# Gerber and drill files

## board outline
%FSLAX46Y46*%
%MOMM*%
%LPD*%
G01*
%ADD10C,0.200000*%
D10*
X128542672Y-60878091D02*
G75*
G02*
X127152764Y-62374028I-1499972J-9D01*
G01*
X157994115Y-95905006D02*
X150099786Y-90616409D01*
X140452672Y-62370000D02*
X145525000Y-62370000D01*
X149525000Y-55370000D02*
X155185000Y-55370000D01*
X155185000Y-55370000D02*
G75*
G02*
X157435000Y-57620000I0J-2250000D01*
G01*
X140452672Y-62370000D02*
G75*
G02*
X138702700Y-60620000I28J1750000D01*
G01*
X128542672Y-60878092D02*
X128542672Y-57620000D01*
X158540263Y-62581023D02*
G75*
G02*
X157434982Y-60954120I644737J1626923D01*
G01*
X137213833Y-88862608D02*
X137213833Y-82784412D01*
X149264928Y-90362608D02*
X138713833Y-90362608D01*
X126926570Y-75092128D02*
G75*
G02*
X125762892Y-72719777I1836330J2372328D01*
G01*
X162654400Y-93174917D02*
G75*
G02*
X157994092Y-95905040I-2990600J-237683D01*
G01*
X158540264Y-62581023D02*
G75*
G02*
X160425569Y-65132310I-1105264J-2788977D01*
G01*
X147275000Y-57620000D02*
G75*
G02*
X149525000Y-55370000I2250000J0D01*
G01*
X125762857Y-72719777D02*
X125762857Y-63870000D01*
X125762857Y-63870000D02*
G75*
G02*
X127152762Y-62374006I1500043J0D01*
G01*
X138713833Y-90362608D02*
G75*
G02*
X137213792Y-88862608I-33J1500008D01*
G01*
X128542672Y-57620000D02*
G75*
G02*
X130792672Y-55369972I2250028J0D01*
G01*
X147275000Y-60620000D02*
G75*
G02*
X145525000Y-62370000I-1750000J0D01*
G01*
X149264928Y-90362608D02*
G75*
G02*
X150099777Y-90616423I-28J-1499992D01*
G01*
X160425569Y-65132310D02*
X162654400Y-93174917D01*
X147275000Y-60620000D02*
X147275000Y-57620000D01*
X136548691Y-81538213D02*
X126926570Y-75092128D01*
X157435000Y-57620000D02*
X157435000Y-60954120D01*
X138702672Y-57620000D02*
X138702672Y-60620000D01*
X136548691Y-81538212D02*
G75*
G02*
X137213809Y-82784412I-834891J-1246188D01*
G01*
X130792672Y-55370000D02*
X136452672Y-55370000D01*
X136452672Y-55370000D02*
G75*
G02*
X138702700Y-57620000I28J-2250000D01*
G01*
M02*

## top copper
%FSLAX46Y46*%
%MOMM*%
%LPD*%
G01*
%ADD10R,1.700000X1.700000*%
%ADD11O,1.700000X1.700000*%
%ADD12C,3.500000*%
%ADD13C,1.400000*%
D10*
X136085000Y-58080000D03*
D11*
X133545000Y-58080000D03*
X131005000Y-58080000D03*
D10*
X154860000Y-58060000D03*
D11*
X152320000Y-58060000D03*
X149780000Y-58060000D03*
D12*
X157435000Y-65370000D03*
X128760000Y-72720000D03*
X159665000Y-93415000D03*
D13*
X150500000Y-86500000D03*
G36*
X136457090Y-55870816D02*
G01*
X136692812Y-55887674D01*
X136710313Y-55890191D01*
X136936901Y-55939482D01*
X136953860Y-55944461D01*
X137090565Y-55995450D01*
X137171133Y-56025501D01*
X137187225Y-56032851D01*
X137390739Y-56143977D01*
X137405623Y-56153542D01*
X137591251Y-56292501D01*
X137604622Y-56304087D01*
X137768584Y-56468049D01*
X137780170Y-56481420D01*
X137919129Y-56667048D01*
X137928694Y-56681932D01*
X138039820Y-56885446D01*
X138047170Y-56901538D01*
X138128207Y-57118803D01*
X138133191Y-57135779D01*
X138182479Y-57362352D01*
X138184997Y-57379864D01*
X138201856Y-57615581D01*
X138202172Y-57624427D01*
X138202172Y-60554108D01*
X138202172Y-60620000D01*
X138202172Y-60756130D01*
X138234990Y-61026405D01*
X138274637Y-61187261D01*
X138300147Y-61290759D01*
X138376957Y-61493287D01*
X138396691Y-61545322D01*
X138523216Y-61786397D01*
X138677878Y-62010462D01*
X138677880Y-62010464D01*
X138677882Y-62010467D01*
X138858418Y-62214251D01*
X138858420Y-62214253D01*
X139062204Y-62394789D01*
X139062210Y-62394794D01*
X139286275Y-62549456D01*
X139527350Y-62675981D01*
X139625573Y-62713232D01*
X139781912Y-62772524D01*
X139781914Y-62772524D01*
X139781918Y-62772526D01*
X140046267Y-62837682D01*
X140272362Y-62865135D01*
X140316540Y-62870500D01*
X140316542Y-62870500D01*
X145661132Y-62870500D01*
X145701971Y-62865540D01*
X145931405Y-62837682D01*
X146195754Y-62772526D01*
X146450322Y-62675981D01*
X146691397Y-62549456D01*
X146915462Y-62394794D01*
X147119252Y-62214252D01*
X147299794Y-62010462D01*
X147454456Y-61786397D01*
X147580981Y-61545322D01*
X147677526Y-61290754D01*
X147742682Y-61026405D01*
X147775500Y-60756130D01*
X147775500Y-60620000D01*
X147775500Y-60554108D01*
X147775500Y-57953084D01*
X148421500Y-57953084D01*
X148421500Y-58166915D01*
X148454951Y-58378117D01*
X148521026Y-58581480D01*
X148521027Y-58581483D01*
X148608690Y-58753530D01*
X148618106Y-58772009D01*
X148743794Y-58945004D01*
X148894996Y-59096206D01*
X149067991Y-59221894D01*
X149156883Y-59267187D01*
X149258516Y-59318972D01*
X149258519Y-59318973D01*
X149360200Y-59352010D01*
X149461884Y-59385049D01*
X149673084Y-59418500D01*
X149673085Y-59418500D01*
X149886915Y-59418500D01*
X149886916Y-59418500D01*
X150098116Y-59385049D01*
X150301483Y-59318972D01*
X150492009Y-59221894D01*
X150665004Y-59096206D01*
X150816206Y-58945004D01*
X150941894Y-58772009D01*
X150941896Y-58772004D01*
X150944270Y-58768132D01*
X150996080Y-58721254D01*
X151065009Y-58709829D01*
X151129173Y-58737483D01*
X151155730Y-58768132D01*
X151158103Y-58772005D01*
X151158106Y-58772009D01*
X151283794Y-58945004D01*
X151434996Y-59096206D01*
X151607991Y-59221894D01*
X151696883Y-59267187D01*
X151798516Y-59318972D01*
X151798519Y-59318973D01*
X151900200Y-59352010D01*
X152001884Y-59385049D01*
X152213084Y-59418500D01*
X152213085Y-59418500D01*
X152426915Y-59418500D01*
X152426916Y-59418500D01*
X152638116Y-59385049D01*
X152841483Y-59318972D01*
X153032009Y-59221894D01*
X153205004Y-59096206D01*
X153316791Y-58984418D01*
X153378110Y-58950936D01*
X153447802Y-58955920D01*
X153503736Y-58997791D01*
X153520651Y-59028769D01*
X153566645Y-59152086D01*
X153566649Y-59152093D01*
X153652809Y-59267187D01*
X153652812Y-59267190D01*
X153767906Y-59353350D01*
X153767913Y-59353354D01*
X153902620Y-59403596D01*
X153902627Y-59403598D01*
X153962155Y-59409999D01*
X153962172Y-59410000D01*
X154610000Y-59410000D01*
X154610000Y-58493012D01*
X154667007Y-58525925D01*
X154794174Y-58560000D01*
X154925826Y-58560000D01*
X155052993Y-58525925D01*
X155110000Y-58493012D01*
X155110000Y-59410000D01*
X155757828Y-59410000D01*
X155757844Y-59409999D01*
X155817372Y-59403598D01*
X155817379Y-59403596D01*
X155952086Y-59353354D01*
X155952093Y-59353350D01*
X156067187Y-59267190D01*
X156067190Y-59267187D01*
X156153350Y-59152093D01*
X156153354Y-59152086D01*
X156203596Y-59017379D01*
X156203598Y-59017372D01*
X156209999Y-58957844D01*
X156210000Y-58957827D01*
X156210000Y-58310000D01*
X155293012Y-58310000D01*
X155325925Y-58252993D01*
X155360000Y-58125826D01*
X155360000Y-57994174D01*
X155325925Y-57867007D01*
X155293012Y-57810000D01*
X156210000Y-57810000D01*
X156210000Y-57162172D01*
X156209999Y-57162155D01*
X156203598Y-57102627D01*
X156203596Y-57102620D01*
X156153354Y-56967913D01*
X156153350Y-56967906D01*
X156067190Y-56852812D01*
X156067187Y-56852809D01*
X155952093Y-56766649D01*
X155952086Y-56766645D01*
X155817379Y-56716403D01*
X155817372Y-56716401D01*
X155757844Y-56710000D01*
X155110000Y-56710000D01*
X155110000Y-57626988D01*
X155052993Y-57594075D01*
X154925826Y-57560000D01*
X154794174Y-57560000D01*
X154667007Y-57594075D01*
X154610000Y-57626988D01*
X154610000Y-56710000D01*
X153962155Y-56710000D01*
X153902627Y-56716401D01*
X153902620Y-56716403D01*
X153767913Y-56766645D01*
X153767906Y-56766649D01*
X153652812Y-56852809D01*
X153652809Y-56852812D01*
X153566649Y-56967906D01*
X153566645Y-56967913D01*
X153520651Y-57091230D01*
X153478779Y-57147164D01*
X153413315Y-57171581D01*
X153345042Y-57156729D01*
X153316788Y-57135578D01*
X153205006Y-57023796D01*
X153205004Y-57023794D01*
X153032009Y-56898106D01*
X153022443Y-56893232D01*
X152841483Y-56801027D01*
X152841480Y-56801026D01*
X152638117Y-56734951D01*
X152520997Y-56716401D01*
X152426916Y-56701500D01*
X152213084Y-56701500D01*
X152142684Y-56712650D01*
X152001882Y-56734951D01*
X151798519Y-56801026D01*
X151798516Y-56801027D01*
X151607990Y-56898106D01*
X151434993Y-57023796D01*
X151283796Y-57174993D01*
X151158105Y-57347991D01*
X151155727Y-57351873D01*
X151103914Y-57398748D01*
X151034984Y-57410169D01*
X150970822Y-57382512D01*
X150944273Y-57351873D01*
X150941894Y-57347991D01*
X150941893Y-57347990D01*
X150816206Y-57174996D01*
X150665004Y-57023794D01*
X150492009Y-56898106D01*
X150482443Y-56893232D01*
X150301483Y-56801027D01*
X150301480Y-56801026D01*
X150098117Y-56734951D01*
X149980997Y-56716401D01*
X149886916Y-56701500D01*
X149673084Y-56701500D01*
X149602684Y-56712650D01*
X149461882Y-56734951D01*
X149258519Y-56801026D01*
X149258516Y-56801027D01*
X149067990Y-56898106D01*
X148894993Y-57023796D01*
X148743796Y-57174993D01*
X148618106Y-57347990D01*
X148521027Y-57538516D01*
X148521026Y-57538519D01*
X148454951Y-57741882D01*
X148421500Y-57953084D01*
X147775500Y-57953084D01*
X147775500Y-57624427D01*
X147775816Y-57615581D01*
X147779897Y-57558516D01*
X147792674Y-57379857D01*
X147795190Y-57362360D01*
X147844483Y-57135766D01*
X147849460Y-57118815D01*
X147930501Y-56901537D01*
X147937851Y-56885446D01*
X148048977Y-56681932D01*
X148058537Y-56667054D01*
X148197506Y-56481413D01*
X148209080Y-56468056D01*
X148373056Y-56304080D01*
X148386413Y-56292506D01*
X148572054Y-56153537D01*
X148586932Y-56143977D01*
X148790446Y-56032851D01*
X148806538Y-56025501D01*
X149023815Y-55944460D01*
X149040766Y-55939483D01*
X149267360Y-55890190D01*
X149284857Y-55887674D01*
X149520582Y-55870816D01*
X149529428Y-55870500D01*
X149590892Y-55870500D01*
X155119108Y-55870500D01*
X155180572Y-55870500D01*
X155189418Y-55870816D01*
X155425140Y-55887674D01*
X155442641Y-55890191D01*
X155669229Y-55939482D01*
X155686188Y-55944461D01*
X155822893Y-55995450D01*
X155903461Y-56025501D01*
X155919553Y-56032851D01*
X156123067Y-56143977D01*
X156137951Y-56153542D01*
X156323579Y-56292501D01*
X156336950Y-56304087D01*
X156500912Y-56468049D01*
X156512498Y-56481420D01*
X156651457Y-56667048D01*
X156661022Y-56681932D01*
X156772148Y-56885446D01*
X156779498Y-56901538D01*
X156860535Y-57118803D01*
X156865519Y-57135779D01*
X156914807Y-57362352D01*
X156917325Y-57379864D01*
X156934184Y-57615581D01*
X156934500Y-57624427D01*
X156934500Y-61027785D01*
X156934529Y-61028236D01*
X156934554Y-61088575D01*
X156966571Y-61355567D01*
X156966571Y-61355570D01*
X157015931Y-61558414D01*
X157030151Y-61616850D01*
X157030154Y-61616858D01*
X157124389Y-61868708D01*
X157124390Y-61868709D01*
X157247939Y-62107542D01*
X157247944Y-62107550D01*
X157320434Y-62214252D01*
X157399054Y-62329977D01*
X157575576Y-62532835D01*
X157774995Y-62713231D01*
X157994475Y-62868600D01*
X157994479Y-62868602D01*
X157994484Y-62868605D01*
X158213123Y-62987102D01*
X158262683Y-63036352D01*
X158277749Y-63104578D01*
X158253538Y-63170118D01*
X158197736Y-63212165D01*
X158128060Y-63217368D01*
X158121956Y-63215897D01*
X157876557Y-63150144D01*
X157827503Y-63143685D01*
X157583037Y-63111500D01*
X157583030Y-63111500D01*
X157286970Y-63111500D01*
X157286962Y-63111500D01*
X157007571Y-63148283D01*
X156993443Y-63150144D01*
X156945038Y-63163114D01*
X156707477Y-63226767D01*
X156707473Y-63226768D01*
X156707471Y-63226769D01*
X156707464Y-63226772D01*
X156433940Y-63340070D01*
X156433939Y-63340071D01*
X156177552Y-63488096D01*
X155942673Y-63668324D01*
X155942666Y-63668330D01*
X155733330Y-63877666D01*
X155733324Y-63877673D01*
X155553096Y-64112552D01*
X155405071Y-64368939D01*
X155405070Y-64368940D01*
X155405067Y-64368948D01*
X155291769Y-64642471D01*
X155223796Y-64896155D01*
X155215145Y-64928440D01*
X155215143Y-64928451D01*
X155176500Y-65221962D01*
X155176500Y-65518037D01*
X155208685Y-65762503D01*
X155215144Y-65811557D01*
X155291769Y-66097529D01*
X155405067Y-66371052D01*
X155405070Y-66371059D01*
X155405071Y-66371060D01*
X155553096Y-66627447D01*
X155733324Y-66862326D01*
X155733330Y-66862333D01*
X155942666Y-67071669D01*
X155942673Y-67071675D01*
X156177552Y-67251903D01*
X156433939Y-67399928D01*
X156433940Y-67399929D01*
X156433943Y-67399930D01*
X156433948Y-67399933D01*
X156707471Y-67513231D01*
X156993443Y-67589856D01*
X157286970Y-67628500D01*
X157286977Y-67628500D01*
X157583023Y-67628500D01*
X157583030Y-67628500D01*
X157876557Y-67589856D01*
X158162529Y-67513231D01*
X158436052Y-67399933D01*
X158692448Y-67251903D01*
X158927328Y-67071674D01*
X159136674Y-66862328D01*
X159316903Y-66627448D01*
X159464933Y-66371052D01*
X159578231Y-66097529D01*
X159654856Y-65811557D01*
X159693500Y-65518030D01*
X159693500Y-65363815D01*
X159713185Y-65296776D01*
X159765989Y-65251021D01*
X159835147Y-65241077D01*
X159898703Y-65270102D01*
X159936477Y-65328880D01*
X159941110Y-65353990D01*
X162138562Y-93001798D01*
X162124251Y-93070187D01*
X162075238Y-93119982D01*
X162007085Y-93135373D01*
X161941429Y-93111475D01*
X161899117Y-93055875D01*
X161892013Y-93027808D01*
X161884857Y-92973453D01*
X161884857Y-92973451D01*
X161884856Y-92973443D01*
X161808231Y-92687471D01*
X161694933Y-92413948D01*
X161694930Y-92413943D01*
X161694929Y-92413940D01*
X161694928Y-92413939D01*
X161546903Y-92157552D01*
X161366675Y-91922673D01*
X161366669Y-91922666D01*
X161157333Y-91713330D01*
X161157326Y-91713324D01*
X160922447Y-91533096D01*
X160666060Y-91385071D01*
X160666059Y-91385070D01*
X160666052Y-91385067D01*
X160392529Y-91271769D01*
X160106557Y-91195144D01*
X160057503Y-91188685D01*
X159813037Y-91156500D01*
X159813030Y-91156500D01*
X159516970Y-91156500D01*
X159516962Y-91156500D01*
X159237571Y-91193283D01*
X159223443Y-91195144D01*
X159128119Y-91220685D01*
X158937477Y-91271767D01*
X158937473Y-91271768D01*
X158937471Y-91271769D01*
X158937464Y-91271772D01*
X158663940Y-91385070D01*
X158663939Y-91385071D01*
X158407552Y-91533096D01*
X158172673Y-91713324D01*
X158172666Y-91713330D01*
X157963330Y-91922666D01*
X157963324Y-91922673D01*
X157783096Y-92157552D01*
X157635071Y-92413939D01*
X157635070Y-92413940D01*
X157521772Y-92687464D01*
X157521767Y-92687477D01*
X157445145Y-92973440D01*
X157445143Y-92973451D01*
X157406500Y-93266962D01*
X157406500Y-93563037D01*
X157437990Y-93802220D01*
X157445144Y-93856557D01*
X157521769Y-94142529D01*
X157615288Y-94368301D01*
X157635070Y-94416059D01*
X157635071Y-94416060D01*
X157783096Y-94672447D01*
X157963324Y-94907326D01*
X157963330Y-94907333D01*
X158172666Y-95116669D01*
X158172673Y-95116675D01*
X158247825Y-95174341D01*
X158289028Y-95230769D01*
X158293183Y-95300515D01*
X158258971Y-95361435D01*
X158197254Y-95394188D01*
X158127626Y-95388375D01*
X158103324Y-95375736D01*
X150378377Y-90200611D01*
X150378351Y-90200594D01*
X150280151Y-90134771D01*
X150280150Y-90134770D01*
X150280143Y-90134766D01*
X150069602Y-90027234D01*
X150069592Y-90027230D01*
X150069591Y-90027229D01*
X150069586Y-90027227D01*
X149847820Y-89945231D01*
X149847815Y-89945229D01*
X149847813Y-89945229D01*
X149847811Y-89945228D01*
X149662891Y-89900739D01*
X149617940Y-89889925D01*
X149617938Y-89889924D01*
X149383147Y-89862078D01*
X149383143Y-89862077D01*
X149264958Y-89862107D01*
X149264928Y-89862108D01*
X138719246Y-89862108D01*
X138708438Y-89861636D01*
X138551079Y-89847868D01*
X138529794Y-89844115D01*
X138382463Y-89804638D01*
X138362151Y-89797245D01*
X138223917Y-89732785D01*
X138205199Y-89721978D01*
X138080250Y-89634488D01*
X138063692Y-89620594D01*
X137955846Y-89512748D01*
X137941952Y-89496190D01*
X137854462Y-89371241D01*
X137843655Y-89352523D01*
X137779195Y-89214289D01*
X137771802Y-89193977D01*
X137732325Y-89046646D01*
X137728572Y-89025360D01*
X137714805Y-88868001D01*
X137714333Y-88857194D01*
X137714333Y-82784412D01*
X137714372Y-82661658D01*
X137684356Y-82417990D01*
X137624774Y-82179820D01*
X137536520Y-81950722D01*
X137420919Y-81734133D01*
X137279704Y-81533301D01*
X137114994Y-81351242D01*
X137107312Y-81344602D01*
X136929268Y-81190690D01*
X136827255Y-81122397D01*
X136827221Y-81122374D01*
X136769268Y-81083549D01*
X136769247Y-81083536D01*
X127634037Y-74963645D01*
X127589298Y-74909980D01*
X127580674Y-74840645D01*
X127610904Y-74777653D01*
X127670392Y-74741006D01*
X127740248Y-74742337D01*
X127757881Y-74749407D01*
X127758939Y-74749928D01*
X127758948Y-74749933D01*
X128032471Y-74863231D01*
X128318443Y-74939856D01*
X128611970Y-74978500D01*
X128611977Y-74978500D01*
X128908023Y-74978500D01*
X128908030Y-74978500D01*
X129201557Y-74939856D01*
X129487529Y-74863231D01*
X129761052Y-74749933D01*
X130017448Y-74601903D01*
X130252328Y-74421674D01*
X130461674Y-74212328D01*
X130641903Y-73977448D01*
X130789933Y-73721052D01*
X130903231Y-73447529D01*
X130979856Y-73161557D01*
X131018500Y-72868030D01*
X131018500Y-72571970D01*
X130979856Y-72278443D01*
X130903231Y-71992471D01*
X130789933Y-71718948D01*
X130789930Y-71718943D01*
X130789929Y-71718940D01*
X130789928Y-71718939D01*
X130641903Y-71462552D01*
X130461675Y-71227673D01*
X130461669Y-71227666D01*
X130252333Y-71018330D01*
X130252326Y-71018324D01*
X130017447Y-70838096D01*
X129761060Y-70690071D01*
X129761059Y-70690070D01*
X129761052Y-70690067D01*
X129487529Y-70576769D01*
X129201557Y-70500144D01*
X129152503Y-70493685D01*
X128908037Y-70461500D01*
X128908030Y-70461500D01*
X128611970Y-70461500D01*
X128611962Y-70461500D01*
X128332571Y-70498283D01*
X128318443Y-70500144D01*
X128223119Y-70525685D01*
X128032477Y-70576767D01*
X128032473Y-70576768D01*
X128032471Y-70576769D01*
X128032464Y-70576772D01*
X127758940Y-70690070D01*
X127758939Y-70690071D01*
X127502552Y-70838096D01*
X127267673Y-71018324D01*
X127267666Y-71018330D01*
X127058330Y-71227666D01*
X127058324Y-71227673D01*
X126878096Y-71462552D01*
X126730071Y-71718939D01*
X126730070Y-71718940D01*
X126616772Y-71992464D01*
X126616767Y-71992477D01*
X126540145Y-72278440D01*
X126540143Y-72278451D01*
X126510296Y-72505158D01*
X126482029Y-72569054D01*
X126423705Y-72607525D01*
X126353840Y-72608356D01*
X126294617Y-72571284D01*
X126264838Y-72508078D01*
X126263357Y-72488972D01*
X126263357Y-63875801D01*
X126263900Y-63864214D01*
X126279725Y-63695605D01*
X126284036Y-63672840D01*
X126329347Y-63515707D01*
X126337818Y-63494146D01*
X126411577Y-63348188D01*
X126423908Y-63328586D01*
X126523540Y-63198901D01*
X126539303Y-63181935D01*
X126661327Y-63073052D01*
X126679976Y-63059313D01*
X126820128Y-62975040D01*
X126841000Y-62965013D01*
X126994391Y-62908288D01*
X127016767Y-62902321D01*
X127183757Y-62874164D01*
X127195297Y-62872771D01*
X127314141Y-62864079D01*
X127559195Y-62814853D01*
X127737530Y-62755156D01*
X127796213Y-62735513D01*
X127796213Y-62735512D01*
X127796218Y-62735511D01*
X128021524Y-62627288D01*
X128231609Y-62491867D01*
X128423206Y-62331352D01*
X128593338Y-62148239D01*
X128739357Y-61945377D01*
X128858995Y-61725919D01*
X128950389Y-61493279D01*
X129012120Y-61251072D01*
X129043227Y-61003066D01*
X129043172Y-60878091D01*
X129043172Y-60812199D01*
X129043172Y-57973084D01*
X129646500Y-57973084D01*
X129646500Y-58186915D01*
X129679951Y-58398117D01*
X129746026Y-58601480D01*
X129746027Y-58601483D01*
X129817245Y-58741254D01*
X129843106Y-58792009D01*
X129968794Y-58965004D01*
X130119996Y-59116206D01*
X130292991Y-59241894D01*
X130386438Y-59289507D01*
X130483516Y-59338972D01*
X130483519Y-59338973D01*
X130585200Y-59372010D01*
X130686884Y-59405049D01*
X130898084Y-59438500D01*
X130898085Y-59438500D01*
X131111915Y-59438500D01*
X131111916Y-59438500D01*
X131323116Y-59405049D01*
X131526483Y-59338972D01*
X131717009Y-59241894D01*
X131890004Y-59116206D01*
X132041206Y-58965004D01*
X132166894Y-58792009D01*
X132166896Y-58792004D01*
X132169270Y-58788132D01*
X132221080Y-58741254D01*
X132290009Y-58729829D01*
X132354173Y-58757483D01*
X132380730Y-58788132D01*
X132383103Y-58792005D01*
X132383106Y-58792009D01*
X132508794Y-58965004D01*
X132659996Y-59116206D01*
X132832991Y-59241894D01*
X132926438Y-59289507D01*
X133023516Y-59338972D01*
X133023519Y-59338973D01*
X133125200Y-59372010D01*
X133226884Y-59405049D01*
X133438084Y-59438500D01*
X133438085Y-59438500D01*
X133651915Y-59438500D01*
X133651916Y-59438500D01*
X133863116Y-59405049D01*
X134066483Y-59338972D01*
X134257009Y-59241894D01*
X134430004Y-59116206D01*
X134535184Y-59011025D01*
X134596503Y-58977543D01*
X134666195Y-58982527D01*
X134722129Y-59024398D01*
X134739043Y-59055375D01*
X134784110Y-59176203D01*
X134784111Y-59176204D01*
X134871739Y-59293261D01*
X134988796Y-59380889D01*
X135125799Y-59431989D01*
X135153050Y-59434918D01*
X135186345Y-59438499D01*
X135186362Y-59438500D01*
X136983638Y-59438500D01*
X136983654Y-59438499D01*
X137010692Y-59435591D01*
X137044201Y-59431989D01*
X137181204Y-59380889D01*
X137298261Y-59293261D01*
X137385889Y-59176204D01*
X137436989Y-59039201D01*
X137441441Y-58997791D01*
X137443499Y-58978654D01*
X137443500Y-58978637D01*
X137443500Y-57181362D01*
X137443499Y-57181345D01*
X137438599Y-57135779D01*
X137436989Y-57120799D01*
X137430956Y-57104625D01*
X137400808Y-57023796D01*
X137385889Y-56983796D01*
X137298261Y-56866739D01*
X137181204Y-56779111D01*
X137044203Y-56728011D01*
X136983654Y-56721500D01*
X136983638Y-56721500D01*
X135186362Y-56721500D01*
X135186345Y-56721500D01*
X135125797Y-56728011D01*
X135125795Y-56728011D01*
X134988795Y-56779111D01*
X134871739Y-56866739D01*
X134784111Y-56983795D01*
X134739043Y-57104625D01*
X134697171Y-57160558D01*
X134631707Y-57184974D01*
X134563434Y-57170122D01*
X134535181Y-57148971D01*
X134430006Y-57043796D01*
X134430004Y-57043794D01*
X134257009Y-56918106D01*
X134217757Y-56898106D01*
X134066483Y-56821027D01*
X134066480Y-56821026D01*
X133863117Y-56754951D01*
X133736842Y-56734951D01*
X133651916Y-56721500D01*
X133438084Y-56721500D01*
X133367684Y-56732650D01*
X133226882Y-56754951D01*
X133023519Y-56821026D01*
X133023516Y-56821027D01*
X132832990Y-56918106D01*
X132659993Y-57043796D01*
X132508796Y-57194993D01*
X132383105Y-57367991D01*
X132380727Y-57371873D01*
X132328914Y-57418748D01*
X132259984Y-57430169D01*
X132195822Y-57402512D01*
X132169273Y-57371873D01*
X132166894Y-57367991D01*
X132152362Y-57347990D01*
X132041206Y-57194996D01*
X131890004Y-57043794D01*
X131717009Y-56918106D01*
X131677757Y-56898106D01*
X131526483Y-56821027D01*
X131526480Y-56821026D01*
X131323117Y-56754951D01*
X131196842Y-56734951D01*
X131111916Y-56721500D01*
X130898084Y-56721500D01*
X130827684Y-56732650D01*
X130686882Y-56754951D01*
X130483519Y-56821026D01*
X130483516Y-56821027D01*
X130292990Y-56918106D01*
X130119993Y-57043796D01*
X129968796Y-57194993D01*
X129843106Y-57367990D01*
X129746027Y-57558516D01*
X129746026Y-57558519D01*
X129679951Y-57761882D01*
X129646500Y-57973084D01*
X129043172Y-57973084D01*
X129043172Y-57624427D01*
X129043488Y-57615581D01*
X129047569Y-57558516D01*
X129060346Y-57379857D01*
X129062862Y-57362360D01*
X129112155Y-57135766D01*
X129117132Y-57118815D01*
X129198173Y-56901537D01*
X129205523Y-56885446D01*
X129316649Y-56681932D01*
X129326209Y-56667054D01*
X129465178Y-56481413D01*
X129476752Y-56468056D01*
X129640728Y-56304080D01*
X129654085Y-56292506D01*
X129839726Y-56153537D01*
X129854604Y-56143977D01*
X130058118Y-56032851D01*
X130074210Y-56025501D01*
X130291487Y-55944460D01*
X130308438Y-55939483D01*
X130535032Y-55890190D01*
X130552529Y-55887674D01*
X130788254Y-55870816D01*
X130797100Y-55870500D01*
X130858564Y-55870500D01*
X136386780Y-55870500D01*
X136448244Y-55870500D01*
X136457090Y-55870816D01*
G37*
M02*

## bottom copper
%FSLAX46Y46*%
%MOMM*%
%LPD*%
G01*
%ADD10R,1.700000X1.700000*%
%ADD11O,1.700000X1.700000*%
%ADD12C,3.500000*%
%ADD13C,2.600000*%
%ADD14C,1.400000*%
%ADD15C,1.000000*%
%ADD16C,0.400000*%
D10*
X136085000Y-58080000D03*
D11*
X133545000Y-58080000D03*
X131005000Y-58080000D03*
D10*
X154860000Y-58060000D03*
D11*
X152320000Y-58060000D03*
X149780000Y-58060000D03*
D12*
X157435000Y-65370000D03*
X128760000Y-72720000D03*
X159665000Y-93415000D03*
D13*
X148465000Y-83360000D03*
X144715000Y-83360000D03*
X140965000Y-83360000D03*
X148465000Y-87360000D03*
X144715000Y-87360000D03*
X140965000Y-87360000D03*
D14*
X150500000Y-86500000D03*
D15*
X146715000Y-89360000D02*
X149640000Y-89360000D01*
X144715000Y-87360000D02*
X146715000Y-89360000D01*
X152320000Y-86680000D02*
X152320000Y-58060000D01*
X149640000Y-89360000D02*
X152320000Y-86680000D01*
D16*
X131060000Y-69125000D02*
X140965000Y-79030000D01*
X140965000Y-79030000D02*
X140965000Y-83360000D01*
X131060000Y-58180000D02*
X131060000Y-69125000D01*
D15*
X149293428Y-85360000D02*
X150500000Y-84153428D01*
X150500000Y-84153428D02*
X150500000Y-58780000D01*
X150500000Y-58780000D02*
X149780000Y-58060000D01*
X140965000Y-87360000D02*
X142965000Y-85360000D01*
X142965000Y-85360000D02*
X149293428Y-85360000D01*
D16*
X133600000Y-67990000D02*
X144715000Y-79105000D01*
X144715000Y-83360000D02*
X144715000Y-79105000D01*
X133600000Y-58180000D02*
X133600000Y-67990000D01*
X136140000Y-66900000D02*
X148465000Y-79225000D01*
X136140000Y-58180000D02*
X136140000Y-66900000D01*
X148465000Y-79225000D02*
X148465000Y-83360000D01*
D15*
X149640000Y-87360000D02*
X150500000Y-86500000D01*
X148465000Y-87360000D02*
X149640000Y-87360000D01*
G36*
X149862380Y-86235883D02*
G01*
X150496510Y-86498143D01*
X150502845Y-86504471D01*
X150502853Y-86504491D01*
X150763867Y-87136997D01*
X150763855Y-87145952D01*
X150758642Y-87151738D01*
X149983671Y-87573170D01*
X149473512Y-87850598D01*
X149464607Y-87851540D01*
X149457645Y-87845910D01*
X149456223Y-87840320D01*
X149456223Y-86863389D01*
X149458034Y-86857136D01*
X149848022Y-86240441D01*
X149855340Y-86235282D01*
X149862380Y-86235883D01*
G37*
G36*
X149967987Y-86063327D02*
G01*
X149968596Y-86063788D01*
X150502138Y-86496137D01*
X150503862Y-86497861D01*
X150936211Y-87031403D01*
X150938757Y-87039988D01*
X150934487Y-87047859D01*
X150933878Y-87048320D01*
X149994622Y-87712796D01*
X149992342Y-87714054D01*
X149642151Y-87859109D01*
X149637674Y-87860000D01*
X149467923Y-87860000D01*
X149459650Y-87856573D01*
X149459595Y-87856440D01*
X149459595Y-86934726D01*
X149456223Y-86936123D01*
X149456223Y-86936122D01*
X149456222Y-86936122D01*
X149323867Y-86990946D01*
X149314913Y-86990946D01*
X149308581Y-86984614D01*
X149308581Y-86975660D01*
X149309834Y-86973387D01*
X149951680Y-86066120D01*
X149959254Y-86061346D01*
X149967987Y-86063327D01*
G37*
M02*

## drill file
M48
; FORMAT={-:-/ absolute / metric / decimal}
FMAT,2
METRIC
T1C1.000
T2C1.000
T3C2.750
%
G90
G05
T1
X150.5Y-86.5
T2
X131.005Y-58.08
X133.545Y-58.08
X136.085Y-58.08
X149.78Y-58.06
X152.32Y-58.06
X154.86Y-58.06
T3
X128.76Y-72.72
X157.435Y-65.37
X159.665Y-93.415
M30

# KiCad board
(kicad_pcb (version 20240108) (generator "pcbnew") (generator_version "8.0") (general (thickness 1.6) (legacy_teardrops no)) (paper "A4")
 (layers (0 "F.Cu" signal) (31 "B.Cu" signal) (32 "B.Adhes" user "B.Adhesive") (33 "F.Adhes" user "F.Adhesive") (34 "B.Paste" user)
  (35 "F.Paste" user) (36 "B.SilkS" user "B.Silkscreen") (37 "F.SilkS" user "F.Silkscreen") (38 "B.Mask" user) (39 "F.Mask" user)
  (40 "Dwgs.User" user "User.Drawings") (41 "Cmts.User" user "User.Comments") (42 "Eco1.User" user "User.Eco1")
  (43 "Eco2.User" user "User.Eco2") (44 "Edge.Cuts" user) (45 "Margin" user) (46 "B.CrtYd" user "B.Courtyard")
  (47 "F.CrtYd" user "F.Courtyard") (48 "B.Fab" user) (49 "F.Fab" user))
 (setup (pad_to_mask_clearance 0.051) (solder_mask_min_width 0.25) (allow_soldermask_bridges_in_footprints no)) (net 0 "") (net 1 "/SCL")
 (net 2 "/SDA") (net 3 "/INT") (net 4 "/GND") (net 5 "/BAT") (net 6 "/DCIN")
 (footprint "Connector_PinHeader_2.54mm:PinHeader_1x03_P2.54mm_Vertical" (layer "F.Cu") (at 136.085 58.08 -90)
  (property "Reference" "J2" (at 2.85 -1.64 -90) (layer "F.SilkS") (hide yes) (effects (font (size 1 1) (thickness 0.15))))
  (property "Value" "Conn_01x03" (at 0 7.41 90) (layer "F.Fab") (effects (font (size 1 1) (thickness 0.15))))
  (pad "1" thru_hole rect (at 0 0 270) (size 1.7 1.7) (drill 1) (layers "*.Cu" "*.Mask") (remove_unused_layers no) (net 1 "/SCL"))
  (pad "2" thru_hole oval (at 0 2.54 270) (size 1.7 1.7) (drill 1) (layers "*.Cu" "*.Mask") (remove_unused_layers no) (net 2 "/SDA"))
  (pad "3" thru_hole oval (at 0 5.08 270) (size 1.7 1.7) (drill 1) (layers "*.Cu" "*.Mask") (remove_unused_layers no) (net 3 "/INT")))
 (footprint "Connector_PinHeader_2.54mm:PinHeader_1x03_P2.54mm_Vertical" (layer "F.Cu") (at 154.86 58.06 -90)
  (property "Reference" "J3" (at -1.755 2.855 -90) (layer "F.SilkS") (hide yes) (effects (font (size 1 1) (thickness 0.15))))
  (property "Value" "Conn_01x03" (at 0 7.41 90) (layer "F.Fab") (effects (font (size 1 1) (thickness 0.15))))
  (pad "1" thru_hole rect (at 0 0 270) (size 1.7 1.7) (drill 1) (layers "*.Cu" "*.Mask") (remove_unused_layers no) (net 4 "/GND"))
  (pad "2" thru_hole oval (at 0 2.54 270) (size 1.7 1.7) (drill 1) (layers "*.Cu" "*.Mask") (remove_unused_layers no) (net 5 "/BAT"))
  (pad "3" thru_hole oval (at 0 5.08 270) (size 1.7 1.7) (drill 1) (layers "*.Cu" "*.Mask") (remove_unused_layers no) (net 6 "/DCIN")))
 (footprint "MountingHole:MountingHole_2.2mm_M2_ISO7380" (layer "F.Cu") (at 157.435 65.37)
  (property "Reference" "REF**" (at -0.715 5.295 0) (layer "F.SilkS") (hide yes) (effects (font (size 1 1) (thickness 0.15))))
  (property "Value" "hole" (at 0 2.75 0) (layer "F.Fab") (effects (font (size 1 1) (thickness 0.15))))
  (pad "" np_thru_hole circle (at 0 0) (size 3.5 3.5) (drill 2.75) (layers "*.Cu" "*.Mask")))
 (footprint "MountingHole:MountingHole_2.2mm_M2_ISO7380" (layer "F.Cu") (at 128.76 72.72)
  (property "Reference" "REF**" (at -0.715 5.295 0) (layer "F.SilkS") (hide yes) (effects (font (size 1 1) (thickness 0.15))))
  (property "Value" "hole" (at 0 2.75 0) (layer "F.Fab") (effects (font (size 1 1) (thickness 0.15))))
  (pad "" np_thru_hole circle (at 0 0) (size 3.5 3.5) (drill 2.75) (layers "*.Cu" "*.Mask")))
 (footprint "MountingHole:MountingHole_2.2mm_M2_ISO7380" (layer "F.Cu") (at 159.665 93.415)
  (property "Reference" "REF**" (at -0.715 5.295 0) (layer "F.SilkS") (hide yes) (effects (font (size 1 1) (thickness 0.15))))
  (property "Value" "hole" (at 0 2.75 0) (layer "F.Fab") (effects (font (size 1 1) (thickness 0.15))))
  (pad "" np_thru_hole circle (at 0 0) (size 3.5 3.5) (drill 2.75) (layers "*.Cu" "*.Mask")))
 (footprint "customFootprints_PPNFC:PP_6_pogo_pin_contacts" (layer "B.Cu") (at 148.465 83.36 180)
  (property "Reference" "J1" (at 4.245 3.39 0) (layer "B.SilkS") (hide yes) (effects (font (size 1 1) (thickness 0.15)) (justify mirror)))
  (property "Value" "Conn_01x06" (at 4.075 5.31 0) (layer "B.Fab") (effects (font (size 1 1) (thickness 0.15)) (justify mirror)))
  (pad "1" smd circle (at 0 0 180) (size 2.6 2.6) (layers "B.Cu" "B.Paste" "B.Mask") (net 1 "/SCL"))
  (pad "2" smd circle (at 3.75 0 180) (size 2.6 2.6) (layers "B.Cu" "B.Paste" "B.Mask") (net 2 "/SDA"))
  (pad "3" smd circle (at 7.5 0 180) (size 2.6 2.6) (layers "B.Cu" "B.Paste" "B.Mask") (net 3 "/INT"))
  (pad "4" smd circle (at 0 -4 180) (size 2.6 2.6) (layers "B.Cu" "B.Paste" "B.Mask") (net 4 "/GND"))
  (pad "5" smd circle (at 3.75 -4 180) (size 2.6 2.6) (layers "B.Cu" "B.Paste" "B.Mask") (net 5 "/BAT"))
  (pad "6" smd circle (at 7.5 -4 180) (size 2.6 2.6) (layers "B.Cu" "B.Paste" "B.Mask") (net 6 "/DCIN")))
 (gr_arc (start 128.542672 60.878091) (mid 128.141567 61.899086) (end 127.152765 62.374046) (stroke (width 0.2) (type solid))
  (layer "Edge.Cuts"))
 (gr_line (start 157.994115 95.905006) (end 150.099786 90.616409) (stroke (width 0.2) (type solid)) (layer "Edge.Cuts"))
 (gr_line (start 140.452672 62.37) (end 145.525 62.37) (stroke (width 0.2) (type solid)) (layer "Edge.Cuts"))
 (gr_line (start 149.525 55.37) (end 155.185 55.37) (stroke (width 0.2) (type solid)) (layer "Edge.Cuts"))
 (gr_arc (start 155.185 55.37) (mid 156.77599 56.02901) (end 157.435 57.62) (stroke (width 0.2) (type solid)) (layer "Edge.Cuts"))
 (gr_arc (start 140.452672 62.37) (mid 139.215235 61.857437) (end 138.702672 60.62) (stroke (width 0.2) (type solid)) (layer "Edge.Cuts"))
 (gr_line (start 128.542672 60.878092) (end 128.542672 57.62) (stroke (width 0.2) (type solid)) (layer "Edge.Cuts"))
 (gr_arc (start 158.540263 62.581023) (mid 157.737452 61.937535) (end 157.435 60.95412) (stroke (width 0.2) (type solid))
  (layer "Edge.Cuts"))
 (gr_line (start 137.213833 88.862608) (end 137.213833 82.784412) (stroke (width 0.2) (type solid)) (layer "Edge.Cuts"))
 (gr_line (start 149.264928 90.362608) (end 138.713833 90.362608) (stroke (width 0.2) (type solid)) (layer "Edge.Cuts"))
 (gr_arc (start 126.92657 75.092128) (mid 126.069452 74.040977) (end 125.762857 72.719777) (stroke (width 0.2) (type solid))
  (layer "Edge.Cuts"))
 (gr_arc (start 162.6544 93.174917) (mid 161.180244 96.001139) (end 157.994115 95.905006) (stroke (width 0.2) (type solid))
  (layer "Edge.Cuts"))
 (gr_arc (start 158.540264 62.581023) (mid 159.847722 63.587089) (end 160.425569 65.13231) (stroke (width 0.2) (type solid))
  (layer "Edge.Cuts"))
 (gr_arc (start 147.275 57.62) (mid 147.93401 56.02901) (end 149.525 55.37) (stroke (width 0.2) (type solid)) (layer "Edge.Cuts"))
 (gr_line (start 125.762857 72.719777) (end 125.762857 63.87) (stroke (width 0.2) (type solid)) (layer "Edge.Cuts"))
 (gr_arc (start 125.762857 63.87) (mid 126.163963 62.849005) (end 127.152765 62.374046) (stroke (width 0.2) (type solid))
  (layer "Edge.Cuts"))
 (gr_arc (start 138.713833 90.362608) (mid 137.653173 89.923268) (end 137.213833 88.862608) (stroke (width 0.2) (type solid))
  (layer "Edge.Cuts"))
 (gr_arc (start 128.542672 57.62) (mid 129.201682 56.02901) (end 130.792672 55.37) (stroke (width 0.2) (type solid)) (layer "Edge.Cuts"))
 (gr_arc (start 147.275 60.62) (mid 146.762437 61.857437) (end 145.525 62.37) (stroke (width 0.2) (type solid)) (layer "Edge.Cuts"))
 (gr_arc (start 149.264928 90.362608) (mid 149.70122 90.42746) (end 150.099786 90.616409) (stroke (width 0.2) (type solid))
  (layer "Edge.Cuts"))
 (gr_line (start 160.425569 65.13231) (end 162.6544 93.174917) (stroke (width 0.2) (type solid)) (layer "Edge.Cuts"))
 (gr_line (start 147.275 60.62) (end 147.275 57.62) (stroke (width 0.2) (type solid)) (layer "Edge.Cuts"))
 (gr_line (start 136.548691 81.538213) (end 126.92657 75.092128) (stroke (width 0.2) (type solid)) (layer "Edge.Cuts"))
 (gr_line (start 157.435 57.62) (end 157.435 60.95412) (stroke (width 0.2) (type solid)) (layer "Edge.Cuts"))
 (gr_line (start 138.702672 57.62) (end 138.702672 60.62) (stroke (width 0.2) (type solid)) (layer "Edge.Cuts"))
 (gr_arc (start 136.548691 81.538212) (mid 137.037141 82.078114) (end 137.213833 82.784412) (stroke (width 0.2) (type solid))
  (layer "Edge.Cuts"))
 (gr_line (start 130.792672 55.37) (end 136.452672 55.37) (stroke (width 0.2) (type solid)) (layer "Edge.Cuts"))
 (gr_arc (start 136.452672 55.37) (mid 138.043662 56.02901) (end 138.702672 57.62) (stroke (width 0.2) (type solid)) (layer "Edge.Cuts"))
 (segment (start 146.715 89.36) (end 149.64 89.36) (width 1) (layer "B.Cu") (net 5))
 (segment (start 144.715 87.36) (end 146.715 89.36) (width 1) (layer "B.Cu") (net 5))
 (segment (start 152.32 86.68) (end 152.32 58.06) (width 1) (layer "B.Cu") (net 5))
 (segment (start 149.64 89.36) (end 152.32 86.68) (width 1) (layer "B.Cu") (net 5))
 (segment (start 131.06 69.125) (end 140.965 79.03) (width 0.4) (layer "B.Cu") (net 3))
 (segment (start 140.965 79.03) (end 140.965 83.36) (width 0.4) (layer "B.Cu") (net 3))
 (segment (start 131.06 58.18) (end 131.06 69.125) (width 0.4) (layer "B.Cu") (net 3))
 (segment (start 149.293428 85.36) (end 150.5 84.153428) (width 1) (layer "B.Cu") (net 6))
 (segment (start 150.5 84.153428) (end 150.5 58.78) (width 1) (layer "B.Cu") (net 6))
 (segment (start 150.5 58.78) (end 149.78 58.06) (width 1) (layer "B.Cu") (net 6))
 (segment (start 140.965 87.36) (end 142.965 85.36) (width 1) (layer "B.Cu") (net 6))
 (segment (start 142.965 85.36) (end 149.293428 85.36) (width 1) (layer "B.Cu") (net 6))
 (segment (start 133.6 67.99) (end 144.715 79.105) (width 0.4) (layer "B.Cu") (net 2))
 (segment (start 144.715 83.36) (end 144.715 79.105) (width 0.4) (layer "B.Cu") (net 2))
 (segment (start 133.6 58.18) (end 133.6 67.99) (width 0.4) (layer "B.Cu") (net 2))
 (segment (start 136.14 66.9) (end 148.465 79.225) (width 0.4) (layer "B.Cu") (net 1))
 (segment (start 136.14 58.18) (end 136.14 66.9) (width 0.4) (layer "B.Cu") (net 1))
 (segment (start 148.465 79.225) (end 148.465 83.36) (width 0.4) (layer "B.Cu") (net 1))
 (via (at 150.5 86.5) (size 1.4) (drill 1) (layers "F.Cu" "B.Cu")
  (teardrops (best_length_ratio 0.5) (max_length 1) (best_width_ratio 1) (max_width 2) (curve_points 0) (filter_ratio 0.9) (enabled yes)
   (allow_two_segments yes) (prefer_zone_connections yes))
  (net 4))
 (segment (start 149.64 87.36) (end 150.5 86.5) (width 1) (layer "B.Cu") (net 4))
 (segment (start 148.465 87.36) (end 149.64 87.36) (width 1) (layer "B.Cu") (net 4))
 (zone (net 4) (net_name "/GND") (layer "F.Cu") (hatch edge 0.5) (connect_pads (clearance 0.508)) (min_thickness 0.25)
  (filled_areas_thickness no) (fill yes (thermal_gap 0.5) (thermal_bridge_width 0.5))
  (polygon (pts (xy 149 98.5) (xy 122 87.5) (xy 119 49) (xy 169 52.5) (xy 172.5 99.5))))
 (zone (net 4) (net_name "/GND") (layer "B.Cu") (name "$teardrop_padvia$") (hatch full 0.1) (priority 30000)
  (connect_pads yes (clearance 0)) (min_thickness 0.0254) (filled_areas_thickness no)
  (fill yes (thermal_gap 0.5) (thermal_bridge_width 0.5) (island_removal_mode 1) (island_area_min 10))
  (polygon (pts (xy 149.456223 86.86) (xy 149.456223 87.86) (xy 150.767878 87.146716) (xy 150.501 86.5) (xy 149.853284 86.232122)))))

